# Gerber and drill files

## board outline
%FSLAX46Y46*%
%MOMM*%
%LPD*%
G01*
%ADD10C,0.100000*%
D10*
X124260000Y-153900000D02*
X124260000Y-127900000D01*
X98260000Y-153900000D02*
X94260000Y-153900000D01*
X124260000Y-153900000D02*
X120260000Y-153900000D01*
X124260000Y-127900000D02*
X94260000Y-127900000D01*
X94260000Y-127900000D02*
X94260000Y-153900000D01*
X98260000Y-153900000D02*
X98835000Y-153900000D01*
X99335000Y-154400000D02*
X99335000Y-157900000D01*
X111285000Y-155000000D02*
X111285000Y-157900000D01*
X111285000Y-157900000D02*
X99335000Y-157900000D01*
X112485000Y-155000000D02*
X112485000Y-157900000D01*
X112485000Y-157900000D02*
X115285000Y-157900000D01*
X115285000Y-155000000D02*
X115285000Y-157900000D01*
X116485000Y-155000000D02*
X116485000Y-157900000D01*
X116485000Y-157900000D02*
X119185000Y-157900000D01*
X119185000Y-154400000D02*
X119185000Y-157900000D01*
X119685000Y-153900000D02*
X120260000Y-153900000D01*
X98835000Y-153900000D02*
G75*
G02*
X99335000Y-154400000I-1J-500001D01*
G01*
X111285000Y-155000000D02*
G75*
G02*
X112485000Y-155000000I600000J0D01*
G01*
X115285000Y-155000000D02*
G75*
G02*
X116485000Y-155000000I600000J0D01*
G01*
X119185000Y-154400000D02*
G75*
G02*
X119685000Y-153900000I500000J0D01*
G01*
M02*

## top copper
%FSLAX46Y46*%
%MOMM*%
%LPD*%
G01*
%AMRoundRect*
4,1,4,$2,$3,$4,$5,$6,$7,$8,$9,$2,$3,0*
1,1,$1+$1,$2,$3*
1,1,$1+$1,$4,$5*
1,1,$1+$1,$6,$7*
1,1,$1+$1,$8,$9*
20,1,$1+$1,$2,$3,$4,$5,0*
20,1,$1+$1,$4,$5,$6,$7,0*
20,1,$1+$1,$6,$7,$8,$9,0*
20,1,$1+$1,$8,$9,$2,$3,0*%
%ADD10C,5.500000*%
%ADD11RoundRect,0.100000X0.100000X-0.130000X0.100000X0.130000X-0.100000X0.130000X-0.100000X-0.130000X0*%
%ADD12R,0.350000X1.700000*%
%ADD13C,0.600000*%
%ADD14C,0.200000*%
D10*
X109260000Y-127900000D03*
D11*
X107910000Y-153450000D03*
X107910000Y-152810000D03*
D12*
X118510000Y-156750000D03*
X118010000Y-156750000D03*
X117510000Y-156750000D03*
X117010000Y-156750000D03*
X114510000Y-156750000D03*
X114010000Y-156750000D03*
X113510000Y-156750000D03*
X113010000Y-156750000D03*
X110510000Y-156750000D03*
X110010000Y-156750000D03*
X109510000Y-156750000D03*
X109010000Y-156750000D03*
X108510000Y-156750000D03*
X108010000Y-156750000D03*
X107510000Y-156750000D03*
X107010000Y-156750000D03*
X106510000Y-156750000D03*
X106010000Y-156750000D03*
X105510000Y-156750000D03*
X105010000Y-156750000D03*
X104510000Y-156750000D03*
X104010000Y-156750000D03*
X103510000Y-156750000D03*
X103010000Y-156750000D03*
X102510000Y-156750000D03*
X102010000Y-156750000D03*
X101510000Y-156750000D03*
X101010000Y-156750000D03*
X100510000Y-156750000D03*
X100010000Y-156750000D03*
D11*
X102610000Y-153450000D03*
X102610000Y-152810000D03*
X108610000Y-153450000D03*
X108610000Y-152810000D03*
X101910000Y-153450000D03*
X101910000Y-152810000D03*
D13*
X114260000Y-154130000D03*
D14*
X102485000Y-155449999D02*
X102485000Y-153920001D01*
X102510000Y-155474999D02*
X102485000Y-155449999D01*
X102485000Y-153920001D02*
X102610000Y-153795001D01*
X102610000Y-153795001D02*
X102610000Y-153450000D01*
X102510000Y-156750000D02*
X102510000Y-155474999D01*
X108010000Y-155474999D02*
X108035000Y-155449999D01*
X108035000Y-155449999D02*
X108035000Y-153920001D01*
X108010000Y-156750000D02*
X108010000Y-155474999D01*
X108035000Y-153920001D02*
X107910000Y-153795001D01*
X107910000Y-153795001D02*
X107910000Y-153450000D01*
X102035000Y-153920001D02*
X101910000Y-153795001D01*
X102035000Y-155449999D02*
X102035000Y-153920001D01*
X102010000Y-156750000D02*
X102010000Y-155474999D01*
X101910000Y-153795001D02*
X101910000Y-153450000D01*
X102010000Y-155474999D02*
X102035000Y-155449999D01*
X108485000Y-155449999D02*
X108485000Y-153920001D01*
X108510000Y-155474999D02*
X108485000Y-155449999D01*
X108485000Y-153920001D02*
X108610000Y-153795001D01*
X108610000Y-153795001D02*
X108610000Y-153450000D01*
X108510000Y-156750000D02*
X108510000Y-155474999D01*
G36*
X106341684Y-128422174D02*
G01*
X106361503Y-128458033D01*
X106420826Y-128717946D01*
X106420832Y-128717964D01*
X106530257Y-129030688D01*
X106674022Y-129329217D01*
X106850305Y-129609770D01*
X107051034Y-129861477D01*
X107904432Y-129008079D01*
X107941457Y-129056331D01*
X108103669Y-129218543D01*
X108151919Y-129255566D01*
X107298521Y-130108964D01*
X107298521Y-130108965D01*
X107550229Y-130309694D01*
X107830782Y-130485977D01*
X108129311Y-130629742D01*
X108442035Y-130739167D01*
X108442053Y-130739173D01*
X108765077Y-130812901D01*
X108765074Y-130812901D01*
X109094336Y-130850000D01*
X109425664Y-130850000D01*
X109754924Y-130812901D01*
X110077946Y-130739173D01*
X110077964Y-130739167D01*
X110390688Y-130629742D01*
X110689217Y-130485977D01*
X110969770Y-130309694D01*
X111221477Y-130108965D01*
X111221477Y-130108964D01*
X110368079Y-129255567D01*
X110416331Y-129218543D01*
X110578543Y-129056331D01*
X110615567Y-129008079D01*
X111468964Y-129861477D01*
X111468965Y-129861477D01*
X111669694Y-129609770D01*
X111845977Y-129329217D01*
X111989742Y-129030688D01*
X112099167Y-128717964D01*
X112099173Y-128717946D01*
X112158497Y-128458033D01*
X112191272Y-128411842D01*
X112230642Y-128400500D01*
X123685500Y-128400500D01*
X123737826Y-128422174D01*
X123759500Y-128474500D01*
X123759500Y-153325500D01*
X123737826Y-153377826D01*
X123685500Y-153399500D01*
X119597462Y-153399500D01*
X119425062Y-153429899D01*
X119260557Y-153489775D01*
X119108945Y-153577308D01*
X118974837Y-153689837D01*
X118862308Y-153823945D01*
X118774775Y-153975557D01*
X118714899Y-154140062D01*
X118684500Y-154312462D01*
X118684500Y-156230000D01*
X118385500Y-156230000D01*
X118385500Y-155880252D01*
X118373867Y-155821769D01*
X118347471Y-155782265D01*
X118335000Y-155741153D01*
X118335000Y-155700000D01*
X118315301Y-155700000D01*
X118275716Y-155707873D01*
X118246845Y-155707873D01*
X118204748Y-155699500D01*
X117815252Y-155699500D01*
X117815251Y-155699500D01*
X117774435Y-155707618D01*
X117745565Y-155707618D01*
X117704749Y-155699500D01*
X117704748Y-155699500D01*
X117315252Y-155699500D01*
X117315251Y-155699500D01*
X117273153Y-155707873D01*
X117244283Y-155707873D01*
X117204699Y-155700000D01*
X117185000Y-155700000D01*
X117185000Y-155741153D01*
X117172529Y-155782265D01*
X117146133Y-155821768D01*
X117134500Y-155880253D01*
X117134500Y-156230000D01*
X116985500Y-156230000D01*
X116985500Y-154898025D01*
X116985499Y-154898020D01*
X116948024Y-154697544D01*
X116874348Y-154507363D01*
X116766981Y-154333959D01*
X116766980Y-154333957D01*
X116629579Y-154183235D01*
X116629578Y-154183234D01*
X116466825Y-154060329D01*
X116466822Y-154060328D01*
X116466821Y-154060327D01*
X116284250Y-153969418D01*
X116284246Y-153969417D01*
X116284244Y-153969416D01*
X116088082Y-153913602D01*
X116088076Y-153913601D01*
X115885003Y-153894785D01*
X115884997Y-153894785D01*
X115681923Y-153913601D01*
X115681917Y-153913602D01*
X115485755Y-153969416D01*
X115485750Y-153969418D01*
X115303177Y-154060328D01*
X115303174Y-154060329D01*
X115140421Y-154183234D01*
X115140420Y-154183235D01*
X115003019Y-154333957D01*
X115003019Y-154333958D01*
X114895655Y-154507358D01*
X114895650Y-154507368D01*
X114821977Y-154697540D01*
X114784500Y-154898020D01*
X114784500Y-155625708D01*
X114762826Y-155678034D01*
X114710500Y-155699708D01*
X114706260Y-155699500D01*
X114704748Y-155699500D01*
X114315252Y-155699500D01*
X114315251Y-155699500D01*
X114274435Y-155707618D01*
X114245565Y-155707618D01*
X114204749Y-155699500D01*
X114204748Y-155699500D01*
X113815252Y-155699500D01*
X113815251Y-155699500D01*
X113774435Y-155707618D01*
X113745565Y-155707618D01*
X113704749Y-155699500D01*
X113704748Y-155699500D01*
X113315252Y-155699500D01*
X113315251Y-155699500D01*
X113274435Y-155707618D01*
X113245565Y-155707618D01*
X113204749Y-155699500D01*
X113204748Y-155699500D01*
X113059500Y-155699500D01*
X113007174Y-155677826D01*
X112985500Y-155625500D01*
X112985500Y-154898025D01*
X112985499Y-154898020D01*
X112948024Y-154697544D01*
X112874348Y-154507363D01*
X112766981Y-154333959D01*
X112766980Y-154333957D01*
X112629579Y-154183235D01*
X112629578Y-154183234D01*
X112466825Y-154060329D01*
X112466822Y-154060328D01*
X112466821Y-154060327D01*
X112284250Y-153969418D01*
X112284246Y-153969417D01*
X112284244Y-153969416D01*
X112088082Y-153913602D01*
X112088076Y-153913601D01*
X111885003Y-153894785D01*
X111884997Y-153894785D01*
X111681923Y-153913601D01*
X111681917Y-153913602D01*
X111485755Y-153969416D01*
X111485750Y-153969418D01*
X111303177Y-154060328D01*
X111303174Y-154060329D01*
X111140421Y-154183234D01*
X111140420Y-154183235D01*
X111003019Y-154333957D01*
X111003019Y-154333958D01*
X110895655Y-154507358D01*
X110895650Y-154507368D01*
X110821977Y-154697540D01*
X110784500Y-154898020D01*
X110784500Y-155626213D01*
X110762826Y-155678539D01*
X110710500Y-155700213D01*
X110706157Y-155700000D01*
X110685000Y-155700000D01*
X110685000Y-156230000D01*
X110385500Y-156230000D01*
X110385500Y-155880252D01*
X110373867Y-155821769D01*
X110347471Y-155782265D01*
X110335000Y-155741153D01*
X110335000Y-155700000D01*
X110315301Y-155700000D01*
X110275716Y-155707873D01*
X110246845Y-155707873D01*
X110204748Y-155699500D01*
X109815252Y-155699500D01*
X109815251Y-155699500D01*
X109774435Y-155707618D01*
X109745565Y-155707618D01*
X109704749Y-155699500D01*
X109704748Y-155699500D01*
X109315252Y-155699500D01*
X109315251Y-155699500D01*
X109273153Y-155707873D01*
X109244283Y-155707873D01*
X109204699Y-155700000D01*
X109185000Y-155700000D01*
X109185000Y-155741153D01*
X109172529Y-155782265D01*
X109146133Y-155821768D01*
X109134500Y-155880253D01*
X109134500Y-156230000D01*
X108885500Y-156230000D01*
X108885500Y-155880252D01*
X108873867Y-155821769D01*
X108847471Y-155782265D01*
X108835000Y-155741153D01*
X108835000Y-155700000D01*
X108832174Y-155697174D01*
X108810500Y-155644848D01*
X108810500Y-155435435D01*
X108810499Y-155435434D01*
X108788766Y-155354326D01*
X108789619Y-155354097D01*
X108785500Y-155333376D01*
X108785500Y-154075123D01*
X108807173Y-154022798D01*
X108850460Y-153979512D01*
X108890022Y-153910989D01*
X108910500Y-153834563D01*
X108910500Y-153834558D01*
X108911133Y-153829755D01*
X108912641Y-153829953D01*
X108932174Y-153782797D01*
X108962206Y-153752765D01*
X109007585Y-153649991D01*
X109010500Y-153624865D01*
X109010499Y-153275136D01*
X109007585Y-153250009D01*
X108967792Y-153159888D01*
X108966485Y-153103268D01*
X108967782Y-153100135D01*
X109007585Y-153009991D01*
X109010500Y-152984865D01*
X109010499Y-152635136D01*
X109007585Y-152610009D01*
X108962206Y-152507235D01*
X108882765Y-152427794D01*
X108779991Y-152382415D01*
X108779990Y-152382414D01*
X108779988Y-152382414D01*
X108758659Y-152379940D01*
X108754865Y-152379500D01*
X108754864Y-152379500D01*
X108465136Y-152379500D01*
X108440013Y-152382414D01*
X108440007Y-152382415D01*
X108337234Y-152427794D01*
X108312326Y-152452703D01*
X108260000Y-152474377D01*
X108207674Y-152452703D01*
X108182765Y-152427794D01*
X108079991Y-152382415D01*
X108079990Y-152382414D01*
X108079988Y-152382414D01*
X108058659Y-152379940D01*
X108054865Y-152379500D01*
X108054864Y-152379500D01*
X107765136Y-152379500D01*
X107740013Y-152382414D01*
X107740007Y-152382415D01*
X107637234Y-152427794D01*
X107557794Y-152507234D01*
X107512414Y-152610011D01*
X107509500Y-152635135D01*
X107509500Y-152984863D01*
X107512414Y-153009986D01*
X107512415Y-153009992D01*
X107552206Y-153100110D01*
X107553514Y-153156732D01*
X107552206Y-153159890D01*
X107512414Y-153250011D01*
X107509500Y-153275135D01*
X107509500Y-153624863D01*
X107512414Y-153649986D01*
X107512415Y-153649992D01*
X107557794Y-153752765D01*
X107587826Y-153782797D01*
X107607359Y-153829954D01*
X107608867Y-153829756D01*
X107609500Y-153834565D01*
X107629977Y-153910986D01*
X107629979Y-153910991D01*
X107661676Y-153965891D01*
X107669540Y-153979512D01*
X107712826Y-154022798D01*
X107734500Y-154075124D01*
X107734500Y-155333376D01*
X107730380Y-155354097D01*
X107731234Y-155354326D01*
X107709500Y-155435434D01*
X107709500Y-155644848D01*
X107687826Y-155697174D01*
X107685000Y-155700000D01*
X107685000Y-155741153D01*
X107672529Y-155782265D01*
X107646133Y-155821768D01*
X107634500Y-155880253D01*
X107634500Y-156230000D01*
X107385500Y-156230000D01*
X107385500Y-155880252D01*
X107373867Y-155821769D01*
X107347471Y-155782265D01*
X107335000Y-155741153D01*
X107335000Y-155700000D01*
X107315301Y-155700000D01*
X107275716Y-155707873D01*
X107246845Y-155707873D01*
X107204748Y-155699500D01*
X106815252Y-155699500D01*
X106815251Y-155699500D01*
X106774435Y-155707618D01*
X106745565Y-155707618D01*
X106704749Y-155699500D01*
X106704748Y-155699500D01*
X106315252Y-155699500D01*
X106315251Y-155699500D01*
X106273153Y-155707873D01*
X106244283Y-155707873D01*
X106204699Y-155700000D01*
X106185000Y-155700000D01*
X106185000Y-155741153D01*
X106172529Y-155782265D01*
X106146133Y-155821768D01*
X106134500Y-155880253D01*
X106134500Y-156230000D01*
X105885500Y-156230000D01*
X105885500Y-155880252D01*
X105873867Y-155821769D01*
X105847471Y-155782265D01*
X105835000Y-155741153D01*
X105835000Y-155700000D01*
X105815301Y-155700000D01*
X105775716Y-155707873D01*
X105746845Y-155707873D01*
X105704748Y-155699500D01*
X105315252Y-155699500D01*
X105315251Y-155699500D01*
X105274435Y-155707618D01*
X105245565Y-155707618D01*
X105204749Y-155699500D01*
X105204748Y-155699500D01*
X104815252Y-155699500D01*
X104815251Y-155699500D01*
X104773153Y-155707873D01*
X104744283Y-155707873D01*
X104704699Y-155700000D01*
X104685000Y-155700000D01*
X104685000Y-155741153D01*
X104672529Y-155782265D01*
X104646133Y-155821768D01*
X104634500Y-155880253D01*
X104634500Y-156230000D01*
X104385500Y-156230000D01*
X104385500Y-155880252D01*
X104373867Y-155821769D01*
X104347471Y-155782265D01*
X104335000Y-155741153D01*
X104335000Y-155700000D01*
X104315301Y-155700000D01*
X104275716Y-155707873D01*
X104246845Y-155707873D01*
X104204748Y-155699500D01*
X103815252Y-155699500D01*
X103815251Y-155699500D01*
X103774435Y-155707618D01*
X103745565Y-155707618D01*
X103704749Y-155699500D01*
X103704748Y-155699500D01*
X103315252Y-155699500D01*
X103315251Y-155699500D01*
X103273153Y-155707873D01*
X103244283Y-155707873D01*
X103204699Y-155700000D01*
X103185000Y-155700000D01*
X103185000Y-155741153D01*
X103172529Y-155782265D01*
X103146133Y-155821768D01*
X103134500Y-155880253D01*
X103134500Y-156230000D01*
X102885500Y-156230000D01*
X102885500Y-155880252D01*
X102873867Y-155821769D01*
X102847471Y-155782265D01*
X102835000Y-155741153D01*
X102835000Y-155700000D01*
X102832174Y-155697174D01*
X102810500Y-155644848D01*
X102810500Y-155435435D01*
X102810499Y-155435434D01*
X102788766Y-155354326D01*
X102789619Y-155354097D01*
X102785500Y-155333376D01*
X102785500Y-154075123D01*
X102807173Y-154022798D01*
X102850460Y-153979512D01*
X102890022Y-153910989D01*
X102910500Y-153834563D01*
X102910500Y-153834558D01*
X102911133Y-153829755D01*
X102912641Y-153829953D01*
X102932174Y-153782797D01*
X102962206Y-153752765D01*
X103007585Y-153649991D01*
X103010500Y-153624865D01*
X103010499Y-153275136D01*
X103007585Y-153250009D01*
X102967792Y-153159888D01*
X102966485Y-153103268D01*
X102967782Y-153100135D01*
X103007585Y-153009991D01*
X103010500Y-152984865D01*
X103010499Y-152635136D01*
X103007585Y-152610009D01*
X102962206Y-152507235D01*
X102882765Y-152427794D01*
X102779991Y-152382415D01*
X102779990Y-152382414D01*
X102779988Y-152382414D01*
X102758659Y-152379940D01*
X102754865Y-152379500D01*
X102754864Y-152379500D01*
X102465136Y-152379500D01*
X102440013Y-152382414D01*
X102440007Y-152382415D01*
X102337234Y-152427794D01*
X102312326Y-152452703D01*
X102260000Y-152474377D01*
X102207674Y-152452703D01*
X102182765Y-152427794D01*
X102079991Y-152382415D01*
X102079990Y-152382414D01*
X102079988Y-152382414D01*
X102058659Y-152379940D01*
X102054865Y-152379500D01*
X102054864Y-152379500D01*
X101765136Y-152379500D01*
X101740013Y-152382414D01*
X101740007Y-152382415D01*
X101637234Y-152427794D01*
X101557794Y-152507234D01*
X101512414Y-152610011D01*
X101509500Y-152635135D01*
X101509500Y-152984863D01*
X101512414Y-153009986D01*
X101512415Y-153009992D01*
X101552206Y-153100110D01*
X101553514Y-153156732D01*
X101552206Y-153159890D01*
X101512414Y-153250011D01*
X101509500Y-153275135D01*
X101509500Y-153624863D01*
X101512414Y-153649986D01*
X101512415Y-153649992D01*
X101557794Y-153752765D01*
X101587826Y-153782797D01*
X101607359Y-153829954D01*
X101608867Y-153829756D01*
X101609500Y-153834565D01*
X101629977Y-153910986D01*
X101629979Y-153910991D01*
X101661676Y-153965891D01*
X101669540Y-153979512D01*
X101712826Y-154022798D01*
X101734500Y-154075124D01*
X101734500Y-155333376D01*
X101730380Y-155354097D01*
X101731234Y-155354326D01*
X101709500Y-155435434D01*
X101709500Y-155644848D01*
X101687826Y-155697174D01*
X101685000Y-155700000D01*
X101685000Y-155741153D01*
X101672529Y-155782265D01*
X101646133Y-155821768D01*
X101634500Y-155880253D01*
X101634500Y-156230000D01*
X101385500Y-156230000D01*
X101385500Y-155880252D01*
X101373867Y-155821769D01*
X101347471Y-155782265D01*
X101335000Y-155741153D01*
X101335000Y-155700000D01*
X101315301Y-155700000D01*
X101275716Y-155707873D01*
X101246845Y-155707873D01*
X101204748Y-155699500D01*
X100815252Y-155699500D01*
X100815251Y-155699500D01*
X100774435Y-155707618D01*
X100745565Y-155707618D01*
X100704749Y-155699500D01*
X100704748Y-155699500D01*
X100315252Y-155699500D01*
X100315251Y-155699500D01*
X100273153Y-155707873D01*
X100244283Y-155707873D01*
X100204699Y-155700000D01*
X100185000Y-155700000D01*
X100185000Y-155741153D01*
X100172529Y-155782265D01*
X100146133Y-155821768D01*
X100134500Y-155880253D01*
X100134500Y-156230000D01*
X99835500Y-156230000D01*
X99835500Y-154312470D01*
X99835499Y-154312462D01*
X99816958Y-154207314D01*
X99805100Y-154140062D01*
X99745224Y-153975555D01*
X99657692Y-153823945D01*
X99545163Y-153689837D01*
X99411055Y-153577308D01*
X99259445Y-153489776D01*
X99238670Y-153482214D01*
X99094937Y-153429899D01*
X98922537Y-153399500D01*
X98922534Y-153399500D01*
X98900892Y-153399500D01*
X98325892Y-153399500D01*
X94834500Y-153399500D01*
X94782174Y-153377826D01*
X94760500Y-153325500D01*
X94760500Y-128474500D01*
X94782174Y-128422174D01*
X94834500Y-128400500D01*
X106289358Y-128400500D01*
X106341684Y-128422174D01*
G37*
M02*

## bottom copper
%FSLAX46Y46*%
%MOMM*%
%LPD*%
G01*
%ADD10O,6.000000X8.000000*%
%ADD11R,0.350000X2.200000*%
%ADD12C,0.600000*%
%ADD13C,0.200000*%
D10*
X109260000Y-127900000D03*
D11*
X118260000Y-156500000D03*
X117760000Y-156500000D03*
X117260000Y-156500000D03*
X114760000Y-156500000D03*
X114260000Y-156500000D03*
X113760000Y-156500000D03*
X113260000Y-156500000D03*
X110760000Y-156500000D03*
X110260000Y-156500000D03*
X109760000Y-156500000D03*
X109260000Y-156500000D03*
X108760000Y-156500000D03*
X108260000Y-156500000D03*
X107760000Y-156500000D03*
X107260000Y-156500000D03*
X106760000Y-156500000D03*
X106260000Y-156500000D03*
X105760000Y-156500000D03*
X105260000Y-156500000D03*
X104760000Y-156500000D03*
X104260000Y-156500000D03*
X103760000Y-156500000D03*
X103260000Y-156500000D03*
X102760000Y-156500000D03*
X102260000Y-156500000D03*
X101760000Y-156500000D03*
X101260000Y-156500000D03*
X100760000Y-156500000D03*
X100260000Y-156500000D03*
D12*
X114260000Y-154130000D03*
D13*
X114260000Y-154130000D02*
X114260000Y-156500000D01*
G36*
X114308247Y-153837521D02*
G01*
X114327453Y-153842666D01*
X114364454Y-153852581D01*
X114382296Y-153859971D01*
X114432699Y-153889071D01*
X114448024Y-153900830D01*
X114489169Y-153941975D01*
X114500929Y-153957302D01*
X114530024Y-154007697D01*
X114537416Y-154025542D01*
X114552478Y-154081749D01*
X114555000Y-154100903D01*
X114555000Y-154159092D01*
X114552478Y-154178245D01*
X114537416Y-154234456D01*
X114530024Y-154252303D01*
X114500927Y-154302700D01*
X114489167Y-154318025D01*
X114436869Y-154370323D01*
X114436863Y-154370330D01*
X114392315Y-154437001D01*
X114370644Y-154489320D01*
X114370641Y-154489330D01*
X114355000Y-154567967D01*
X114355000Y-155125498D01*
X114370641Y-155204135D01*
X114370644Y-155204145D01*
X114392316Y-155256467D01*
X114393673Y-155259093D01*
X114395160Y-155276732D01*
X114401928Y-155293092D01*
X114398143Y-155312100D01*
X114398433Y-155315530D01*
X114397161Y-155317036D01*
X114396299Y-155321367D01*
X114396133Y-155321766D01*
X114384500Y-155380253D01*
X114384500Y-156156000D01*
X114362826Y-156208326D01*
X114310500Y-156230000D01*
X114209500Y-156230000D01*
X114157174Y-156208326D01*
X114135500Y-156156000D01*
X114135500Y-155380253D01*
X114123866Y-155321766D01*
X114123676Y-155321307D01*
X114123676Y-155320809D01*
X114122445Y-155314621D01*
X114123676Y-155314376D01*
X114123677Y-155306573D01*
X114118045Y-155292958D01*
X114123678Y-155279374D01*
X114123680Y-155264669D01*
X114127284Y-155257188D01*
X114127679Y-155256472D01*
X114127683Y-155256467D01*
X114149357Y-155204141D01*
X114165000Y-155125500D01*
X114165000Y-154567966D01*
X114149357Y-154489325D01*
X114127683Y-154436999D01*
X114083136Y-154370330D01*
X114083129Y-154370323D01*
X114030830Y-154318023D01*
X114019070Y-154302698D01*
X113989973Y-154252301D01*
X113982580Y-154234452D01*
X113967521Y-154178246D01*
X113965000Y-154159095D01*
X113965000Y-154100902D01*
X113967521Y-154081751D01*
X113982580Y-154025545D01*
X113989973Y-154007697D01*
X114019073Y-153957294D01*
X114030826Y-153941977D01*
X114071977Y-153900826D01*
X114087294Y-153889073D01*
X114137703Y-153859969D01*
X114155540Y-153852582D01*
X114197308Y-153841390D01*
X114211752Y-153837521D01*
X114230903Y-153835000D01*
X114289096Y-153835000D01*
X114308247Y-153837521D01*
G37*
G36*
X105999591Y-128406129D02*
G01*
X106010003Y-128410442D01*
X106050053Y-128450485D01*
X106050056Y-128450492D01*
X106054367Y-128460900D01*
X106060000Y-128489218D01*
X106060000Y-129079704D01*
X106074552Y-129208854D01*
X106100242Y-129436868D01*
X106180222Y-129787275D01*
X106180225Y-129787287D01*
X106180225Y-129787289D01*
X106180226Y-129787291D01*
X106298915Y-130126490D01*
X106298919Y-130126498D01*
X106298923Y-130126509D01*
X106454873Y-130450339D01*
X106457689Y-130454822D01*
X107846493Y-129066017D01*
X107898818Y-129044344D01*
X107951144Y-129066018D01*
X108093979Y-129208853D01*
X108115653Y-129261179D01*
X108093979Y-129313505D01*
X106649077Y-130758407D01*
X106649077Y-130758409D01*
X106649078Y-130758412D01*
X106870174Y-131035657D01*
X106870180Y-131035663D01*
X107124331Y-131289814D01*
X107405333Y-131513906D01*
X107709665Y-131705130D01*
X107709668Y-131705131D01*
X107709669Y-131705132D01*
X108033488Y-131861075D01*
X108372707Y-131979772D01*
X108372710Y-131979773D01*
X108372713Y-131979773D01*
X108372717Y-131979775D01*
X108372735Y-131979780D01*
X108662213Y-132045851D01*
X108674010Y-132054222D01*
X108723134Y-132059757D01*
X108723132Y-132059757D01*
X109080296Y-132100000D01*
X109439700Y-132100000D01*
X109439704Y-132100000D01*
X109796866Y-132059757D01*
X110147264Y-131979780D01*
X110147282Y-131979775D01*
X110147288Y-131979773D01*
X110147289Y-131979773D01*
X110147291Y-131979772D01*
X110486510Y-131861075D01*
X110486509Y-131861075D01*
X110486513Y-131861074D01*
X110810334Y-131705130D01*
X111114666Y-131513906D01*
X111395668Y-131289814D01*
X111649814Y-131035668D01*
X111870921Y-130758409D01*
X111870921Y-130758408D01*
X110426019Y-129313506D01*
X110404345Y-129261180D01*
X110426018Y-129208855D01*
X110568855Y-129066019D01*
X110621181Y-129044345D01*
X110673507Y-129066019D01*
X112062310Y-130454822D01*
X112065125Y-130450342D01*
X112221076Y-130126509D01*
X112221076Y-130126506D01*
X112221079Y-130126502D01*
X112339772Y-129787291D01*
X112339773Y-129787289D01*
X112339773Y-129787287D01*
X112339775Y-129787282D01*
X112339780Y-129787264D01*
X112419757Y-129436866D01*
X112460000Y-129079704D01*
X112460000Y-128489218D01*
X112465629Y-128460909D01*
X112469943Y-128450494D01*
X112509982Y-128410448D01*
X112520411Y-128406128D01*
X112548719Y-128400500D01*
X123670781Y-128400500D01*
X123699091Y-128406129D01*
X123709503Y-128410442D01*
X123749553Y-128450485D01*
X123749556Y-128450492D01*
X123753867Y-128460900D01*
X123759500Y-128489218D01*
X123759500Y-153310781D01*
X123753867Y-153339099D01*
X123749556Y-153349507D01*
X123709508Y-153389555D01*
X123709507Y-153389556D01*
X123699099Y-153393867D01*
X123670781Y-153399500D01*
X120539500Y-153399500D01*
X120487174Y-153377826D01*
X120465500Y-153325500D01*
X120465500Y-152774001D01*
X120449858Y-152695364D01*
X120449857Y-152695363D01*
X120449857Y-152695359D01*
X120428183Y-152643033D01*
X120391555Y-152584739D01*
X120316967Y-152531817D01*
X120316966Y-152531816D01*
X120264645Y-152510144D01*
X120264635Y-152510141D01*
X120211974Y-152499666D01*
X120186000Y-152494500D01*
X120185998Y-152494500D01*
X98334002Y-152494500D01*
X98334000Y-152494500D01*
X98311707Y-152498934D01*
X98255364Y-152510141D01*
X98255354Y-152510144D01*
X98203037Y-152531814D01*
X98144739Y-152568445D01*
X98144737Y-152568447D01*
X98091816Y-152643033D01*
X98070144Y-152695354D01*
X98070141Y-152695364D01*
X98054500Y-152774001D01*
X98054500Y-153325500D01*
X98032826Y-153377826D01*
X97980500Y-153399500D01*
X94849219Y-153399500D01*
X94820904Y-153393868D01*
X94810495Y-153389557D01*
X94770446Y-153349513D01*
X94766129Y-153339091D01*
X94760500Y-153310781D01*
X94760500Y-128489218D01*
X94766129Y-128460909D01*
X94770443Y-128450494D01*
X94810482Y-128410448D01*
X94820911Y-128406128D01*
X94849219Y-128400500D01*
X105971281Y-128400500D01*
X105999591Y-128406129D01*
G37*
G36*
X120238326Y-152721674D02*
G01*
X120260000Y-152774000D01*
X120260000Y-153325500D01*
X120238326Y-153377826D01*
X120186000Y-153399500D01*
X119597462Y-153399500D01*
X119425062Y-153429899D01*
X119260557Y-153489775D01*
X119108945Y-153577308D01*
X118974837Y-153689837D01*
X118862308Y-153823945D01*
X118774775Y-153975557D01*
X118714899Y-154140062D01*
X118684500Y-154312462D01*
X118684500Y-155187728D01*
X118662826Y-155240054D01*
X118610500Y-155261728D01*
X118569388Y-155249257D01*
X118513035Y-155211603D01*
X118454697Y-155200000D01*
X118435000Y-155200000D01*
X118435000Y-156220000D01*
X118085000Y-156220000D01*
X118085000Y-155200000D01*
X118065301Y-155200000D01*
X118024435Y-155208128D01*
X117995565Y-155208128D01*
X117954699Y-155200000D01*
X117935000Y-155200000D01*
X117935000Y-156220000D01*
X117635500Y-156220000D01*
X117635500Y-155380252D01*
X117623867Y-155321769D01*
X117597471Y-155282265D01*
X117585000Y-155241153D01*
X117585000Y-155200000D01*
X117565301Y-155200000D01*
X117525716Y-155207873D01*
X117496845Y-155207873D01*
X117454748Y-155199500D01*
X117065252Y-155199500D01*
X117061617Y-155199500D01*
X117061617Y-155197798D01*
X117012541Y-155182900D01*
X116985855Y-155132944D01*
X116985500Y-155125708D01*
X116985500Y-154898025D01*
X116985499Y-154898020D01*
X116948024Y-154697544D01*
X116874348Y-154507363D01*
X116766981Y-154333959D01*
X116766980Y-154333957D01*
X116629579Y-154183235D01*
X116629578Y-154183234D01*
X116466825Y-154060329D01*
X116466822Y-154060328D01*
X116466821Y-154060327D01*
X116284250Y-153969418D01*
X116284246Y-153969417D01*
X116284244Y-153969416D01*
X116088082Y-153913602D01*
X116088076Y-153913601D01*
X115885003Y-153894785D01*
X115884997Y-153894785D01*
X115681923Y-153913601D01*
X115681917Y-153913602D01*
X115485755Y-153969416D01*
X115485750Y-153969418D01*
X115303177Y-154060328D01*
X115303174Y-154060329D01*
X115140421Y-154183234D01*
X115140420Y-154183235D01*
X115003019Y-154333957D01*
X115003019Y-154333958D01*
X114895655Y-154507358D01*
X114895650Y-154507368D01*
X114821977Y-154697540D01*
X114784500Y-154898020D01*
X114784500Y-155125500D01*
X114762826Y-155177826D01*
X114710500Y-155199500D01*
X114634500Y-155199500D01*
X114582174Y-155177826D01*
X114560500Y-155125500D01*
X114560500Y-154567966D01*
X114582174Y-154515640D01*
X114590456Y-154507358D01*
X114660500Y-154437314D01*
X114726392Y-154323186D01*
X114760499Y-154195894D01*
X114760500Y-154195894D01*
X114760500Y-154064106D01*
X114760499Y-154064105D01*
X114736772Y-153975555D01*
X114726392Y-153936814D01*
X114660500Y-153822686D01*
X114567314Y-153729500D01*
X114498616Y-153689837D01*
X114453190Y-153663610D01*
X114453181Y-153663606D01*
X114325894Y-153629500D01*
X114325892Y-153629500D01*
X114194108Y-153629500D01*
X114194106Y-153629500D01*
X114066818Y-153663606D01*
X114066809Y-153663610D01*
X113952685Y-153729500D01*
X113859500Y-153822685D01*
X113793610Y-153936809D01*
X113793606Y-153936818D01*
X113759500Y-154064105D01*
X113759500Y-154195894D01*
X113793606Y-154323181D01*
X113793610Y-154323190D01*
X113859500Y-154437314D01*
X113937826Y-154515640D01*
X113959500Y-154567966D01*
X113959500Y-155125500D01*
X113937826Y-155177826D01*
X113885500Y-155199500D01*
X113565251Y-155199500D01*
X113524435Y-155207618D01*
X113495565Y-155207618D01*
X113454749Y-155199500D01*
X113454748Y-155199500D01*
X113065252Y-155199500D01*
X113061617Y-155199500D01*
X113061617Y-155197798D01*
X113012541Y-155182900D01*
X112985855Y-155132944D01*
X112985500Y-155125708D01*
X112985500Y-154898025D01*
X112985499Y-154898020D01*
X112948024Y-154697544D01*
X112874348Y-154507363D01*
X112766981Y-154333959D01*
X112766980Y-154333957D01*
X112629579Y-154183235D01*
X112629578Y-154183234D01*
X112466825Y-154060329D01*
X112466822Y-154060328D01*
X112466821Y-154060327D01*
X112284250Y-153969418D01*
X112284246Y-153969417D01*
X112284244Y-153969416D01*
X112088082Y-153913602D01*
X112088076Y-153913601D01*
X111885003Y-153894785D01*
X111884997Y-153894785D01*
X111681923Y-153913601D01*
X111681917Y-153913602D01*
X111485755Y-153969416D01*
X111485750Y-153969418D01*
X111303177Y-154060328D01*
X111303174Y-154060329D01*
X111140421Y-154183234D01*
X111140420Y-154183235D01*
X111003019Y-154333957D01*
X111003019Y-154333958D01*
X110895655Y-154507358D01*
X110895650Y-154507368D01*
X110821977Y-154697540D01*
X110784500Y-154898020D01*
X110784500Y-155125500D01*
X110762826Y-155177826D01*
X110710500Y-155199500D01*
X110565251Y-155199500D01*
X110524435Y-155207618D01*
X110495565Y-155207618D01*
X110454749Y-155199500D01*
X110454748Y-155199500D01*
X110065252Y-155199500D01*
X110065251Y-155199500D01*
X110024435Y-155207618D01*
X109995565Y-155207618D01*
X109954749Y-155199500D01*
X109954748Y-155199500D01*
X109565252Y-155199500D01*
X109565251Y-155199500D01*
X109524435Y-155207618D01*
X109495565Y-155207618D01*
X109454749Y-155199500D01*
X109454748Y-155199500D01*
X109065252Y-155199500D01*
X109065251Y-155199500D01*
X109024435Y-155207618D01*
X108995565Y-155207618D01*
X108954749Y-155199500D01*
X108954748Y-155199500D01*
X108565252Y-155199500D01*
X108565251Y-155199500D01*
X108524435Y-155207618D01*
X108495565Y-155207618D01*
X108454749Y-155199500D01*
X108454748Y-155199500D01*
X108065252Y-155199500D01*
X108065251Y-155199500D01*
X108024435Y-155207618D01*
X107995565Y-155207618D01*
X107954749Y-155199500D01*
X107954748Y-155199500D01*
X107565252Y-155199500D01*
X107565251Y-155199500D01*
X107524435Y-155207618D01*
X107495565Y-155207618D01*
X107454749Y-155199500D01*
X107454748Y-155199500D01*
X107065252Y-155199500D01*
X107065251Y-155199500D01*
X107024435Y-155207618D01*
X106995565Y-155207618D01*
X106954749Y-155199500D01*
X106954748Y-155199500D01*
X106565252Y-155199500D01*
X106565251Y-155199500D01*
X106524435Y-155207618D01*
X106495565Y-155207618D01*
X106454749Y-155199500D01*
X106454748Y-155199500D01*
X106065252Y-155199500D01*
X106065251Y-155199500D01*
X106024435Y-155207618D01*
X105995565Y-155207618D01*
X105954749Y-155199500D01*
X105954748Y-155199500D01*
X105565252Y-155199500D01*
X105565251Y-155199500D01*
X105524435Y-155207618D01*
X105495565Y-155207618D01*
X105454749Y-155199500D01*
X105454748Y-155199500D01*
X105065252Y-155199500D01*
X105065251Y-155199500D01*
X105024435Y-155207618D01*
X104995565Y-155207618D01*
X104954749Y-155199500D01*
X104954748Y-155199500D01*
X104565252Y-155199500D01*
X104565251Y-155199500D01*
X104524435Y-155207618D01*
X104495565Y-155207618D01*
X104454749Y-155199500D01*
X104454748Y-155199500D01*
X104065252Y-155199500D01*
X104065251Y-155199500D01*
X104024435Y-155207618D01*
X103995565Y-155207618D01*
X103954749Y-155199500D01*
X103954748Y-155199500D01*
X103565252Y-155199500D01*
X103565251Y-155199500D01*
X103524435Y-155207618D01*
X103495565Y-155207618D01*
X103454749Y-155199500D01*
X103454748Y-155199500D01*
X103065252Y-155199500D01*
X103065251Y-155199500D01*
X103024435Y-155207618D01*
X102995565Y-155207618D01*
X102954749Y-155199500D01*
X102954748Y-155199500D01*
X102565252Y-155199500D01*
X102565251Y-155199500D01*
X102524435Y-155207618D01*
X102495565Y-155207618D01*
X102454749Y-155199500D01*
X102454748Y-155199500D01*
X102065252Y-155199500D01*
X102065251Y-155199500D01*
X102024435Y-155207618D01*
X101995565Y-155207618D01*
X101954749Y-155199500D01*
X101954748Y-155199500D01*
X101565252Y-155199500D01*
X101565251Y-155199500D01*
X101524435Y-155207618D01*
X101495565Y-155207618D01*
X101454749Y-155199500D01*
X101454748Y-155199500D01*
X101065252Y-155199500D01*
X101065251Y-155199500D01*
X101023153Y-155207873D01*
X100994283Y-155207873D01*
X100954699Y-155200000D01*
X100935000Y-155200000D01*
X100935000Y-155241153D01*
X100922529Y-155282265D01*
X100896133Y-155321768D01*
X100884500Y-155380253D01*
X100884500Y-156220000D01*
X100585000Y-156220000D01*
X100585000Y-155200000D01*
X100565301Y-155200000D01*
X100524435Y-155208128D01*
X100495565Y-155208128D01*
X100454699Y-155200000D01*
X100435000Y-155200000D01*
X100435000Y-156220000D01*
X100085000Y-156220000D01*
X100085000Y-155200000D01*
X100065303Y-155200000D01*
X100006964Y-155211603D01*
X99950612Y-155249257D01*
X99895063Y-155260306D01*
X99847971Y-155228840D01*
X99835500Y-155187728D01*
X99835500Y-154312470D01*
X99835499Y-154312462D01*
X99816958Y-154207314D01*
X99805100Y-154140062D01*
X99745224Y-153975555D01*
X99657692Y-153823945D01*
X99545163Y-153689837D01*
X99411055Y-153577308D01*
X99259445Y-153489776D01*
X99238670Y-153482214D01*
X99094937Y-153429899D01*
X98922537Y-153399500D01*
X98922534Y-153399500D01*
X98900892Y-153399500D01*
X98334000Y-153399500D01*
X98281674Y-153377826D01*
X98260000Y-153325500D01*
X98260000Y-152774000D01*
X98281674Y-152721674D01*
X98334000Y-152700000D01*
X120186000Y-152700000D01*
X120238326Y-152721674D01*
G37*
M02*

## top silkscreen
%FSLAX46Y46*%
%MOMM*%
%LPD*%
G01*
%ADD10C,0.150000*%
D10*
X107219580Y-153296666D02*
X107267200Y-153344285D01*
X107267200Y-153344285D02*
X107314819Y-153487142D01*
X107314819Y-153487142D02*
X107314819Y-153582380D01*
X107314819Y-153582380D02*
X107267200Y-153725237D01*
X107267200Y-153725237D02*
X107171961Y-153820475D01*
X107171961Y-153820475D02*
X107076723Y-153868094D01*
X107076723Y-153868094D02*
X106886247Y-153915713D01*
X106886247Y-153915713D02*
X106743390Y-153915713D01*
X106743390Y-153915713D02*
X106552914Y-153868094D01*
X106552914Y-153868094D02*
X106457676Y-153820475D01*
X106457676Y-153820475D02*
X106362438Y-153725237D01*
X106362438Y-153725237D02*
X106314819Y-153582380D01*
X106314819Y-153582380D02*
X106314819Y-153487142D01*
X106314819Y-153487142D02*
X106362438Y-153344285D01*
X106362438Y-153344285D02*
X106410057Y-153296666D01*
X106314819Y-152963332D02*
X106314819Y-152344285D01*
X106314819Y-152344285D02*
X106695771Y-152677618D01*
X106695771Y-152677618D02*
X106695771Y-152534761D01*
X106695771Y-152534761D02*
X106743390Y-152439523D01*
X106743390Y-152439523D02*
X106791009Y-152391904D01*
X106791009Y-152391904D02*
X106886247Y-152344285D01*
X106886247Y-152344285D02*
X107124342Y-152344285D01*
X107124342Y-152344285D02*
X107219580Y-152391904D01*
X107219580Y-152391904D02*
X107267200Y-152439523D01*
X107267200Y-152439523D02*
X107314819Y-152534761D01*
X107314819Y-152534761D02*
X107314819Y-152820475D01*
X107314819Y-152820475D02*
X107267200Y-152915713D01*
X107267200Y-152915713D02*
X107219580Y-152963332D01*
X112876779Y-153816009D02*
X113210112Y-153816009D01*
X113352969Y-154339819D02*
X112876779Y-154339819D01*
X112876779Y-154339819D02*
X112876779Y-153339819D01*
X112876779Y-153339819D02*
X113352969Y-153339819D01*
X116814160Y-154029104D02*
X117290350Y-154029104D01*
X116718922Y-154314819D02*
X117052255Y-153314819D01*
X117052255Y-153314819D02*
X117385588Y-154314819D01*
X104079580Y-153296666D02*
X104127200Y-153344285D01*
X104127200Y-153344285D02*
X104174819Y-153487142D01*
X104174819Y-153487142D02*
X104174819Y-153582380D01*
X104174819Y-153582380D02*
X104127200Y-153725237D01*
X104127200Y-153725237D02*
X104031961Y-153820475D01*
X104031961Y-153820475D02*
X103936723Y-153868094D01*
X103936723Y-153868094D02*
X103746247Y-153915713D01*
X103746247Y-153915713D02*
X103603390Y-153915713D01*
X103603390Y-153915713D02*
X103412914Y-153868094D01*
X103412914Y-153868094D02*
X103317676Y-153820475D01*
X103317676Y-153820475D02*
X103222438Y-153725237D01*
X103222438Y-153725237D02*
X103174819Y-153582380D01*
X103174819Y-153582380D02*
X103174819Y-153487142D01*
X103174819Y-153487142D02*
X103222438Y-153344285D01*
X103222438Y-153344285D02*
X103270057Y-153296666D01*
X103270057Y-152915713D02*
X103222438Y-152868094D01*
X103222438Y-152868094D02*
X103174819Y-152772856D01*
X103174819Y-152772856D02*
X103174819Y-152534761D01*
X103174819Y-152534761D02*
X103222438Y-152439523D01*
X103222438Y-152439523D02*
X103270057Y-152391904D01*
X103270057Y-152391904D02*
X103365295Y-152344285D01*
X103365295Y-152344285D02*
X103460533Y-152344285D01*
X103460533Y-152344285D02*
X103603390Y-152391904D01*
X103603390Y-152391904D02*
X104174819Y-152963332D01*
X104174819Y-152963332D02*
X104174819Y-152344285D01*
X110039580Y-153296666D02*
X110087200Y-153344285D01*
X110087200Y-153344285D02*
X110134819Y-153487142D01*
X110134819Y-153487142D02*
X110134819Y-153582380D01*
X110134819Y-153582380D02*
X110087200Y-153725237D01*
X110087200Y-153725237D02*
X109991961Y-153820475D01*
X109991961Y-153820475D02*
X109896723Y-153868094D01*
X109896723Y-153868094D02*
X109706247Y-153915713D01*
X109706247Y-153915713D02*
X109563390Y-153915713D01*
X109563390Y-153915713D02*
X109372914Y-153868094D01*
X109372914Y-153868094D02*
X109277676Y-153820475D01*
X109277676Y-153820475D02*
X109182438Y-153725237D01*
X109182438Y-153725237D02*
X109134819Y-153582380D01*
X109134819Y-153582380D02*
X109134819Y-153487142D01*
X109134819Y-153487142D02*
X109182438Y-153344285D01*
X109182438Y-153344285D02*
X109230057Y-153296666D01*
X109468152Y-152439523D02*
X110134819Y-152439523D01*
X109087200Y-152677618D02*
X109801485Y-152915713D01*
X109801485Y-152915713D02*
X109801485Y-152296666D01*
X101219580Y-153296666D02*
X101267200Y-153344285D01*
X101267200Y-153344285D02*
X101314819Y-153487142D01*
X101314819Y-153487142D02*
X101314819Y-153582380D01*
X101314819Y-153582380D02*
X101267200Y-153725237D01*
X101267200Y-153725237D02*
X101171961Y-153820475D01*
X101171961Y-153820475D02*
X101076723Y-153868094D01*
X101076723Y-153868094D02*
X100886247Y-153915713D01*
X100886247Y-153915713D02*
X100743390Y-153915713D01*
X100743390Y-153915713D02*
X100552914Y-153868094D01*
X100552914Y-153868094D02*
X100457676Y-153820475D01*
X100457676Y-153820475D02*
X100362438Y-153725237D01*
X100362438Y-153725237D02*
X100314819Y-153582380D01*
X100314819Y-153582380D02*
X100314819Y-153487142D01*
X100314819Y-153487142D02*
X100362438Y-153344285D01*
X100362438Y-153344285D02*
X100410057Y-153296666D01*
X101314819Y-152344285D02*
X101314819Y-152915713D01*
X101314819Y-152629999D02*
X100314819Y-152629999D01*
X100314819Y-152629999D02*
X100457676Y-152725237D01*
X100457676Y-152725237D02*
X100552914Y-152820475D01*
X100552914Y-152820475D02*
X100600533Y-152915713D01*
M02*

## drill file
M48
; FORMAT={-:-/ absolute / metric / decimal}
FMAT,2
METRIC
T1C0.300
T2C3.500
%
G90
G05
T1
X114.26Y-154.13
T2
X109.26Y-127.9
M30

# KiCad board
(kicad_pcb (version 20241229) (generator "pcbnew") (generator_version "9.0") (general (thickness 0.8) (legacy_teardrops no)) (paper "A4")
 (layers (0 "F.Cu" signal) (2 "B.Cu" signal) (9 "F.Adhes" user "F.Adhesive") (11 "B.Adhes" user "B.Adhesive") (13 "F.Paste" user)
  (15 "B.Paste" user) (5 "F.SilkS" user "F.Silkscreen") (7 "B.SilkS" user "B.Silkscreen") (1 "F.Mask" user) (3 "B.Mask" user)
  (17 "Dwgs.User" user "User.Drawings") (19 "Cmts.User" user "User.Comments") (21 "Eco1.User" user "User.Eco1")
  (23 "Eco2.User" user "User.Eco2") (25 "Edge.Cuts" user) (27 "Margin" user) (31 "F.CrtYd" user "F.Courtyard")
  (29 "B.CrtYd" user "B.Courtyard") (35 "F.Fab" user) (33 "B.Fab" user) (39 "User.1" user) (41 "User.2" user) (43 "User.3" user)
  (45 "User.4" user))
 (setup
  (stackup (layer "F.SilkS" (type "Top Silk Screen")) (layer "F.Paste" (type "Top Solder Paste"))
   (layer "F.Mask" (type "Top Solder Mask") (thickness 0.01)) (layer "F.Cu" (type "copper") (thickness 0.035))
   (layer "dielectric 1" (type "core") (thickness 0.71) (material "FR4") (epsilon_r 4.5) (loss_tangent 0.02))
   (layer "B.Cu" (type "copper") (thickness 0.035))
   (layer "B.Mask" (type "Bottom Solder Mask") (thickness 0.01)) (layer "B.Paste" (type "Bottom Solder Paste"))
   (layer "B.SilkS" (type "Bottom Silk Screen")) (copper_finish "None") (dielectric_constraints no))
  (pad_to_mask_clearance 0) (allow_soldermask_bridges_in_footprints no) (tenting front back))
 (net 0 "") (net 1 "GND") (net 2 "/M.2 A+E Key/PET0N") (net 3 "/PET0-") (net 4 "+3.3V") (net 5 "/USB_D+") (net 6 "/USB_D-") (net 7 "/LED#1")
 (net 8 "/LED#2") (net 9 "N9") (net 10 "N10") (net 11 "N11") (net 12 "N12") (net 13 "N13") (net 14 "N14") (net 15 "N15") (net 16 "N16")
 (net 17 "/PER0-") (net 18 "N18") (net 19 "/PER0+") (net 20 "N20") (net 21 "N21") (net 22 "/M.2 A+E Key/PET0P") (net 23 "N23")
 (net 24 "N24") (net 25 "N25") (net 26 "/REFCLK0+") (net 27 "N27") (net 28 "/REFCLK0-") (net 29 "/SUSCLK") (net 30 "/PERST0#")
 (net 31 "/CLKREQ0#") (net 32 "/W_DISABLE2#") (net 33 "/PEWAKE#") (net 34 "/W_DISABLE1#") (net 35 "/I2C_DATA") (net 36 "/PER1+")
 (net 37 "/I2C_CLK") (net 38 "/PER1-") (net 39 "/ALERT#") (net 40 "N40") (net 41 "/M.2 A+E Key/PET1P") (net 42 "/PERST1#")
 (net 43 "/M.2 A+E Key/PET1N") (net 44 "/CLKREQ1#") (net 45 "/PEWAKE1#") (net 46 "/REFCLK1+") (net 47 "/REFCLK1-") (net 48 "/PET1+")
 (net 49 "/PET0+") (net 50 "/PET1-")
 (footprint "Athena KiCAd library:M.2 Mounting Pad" (layer "F.Cu") (at 109.26 127.9)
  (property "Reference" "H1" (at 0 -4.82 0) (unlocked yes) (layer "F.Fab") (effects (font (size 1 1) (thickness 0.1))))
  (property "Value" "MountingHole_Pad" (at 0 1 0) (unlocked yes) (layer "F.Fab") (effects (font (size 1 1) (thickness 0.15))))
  (pad "1" thru_hole circle (at 0 0) (size 5.5 5.5) (drill 3.5) (layers "*.Cu" "*.Mask") (remove_unused_layers no) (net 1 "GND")
   (padstack (mode front_inner_back)
    (layer "Inner" (shape circle) (size 5.5 5.5) (zone_connect -1))
    (layer "B.Cu" (shape oval) (size 6 8) (thermal_bridge_angle 45) (zone_connect -1)))))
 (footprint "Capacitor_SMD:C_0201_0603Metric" (layer "F.Cu") (at 107.91 153.13 90)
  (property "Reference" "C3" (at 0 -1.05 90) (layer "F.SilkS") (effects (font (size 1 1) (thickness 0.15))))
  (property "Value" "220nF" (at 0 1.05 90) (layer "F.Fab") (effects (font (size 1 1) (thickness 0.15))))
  (pad "" smd roundrect (at -0.345 0 90) (size 0.318 0.36) (layers "F.Paste") (roundrect_rratio 0.25))
  (pad "" smd roundrect (at 0.345 0 90) (size 0.318 0.36) (layers "F.Paste") (roundrect_rratio 0.25))
  (pad "1" smd roundrect (at -0.32 0 90) (size 0.46 0.4) (layers "F.Cu" "F.Mask") (roundrect_rratio 0.25) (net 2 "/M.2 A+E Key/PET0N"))
  (pad "2" smd roundrect (at 0.32 0 90) (size 0.46 0.4) (layers "F.Cu" "F.Mask") (roundrect_rratio 0.25) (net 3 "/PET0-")))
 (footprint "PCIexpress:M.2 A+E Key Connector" (layer "F.Cu") (at 109.26 156.79)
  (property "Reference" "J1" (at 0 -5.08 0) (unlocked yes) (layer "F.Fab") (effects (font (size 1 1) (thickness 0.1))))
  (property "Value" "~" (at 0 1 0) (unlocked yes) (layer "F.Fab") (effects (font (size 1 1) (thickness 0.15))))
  (fp_line (start -11 -2.89) (end -10.425 -2.89) (stroke (width 0.1) (type default)) (layer "Edge.Cuts"))
  (fp_line (start -9.925 -2.39) (end -9.925 1.11) (stroke (width 0.1) (type default)) (layer "Edge.Cuts"))
  (fp_line (start 2.025 -1.79) (end 2.025 1.11) (stroke (width 0.1) (type default)) (layer "Edge.Cuts"))
  (fp_line (start 2.025 1.11) (end -9.925 1.11) (stroke (width 0.1) (type default)) (layer "Edge.Cuts"))
  (fp_line (start 3.225 -1.79) (end 3.225 1.11) (stroke (width 0.1) (type default)) (layer "Edge.Cuts"))
  (fp_line (start 3.225 1.11) (end 6.025 1.11) (stroke (width 0.1) (type default)) (layer "Edge.Cuts"))
  (fp_line (start 6.025 -1.79) (end 6.025 1.11) (stroke (width 0.1) (type default)) (layer "Edge.Cuts"))
  (fp_line (start 7.225 -1.79) (end 7.225 1.11) (stroke (width 0.1) (type default)) (layer "Edge.Cuts"))
  (fp_line (start 7.225 1.11) (end 9.925 1.11) (stroke (width 0.1) (type default)) (layer "Edge.Cuts"))
  (fp_line (start 9.925 -2.39) (end 9.925 1.11) (stroke (width 0.1) (type default)) (layer "Edge.Cuts"))
  (fp_line (start 10.425 -2.89) (end 11 -2.89) (stroke (width 0.1) (type default)) (layer "Edge.Cuts"))
  (fp_arc (start -10.425 -2.89) (mid -10.071447 -2.743553) (end -9.925 -2.39) (stroke (width 0.1) (type default)) (layer "Edge.Cuts"))
  (fp_arc (start 2.025 -1.79) (mid 2.625 -2.39) (end 3.225 -1.79) (stroke (width 0.1) (type default)) (layer "Edge.Cuts"))
  (fp_arc (start 6.025 -1.79) (mid 6.625 -2.39) (end 7.225 -1.79) (stroke (width 0.1) (type default)) (layer "Edge.Cuts"))
  (fp_arc (start 9.925 -2.39) (mid 10.071447 -2.743553) (end 10.425 -2.89) (stroke (width 0.1) (type default)) (layer "Edge.Cuts"))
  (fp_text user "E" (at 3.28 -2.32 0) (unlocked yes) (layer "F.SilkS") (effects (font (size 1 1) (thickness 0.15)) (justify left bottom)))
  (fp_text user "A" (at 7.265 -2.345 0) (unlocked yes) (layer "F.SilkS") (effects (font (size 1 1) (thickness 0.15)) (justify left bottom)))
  (pad "1" smd rect (at 9.25 -0.04 180) (size 0.35 1.7) (layers "F.Cu") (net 1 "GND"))
  (pad "2" smd rect (at 9 -0.29 180) (size 0.35 2.2) (layers "B.Cu") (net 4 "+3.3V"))
  (pad "3" smd rect (at 8.75 -0.04 180) (size 0.35 1.7) (layers "F.Cu") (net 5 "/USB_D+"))
  (pad "4" smd rect (at 8.5 -0.29 180) (size 0.35 2.2) (layers "B.Cu") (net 4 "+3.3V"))
  (pad "5" smd rect (at 8.25 -0.04 180) (size 0.35 1.7) (layers "F.Cu") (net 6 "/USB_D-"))
  (pad "6" smd rect (at 8 -0.29 180) (size 0.35 2.2) (layers "B.Cu") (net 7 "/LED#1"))
  (pad "7" smd rect (at 7.75 -0.04 180) (size 0.35 1.7) (layers "F.Cu") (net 1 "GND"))
  (pad "16" smd rect (at 5.5 -0.29 180) (size 0.35 2.2) (layers "B.Cu") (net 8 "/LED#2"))
  (pad "17" smd rect (at 5.25 -0.04 180) (size 0.35 1.7) (layers "F.Cu") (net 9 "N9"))
  (pad "18" smd rect (at 5 -0.29 180) (size 0.35 2.2) (layers "B.Cu") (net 1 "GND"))
  (pad "19" smd rect (at 4.75 -0.04 180) (size 0.35 1.7) (layers "F.Cu") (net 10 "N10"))
  (pad "20" smd rect (at 4.5 -0.29 180) (size 0.35 2.2) (layers "B.Cu") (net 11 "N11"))
  (pad "21" smd rect (at 4.25 -0.04 180) (size 0.35 1.7) (layers "F.Cu") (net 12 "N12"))
  (pad "22" smd rect (at 4 -0.29 180) (size 0.35 2.2) (layers "B.Cu") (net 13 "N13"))
  (pad "23" smd rect (at 3.75 -0.04 180) (size 0.35 1.7) (layers "F.Cu") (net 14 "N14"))
  (pad "32" smd rect (at 1.5 -0.29 180) (size 0.35 2.2) (layers "B.Cu") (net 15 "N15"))
  (pad "33" smd rect (at 1.25 -0.04 180) (size 0.35 1.7) (layers "F.Cu") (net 1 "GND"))
  (pad "34" smd rect (at 1 -0.29 180) (size 0.35 2.2) (layers "B.Cu") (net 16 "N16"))
  (pad "35" smd rect (at 0.75 -0.04 180) (size 0.35 1.7) (layers "F.Cu") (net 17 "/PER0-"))
  (pad "36" smd rect (at 0.5 -0.29 180) (size 0.35 2.2) (layers "B.Cu") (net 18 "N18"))
  (pad "37" smd rect (at 0.25 -0.04 180) (size 0.35 1.7) (layers "F.Cu") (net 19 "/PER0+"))
  (pad "38" smd rect (at 0 -0.29 180) (size 0.35 2.2) (layers "B.Cu") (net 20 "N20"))
  (pad "39" smd rect (at -0.25 -0.04 180) (size 0.35 1.7) (layers "F.Cu") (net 1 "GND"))
  (pad "40" smd rect (at -0.5 -0.29 180) (size 0.35 2.2) (layers "B.Cu") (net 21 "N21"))
  (pad "41" smd rect (at -0.75 -0.04 180) (size 0.35 1.7) (layers "F.Cu") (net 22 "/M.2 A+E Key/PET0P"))
  (pad "42" smd rect (at -1 -0.29 180) (size 0.35 2.2) (layers "B.Cu") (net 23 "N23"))
  (pad "43" smd rect (at -1.25 -0.04 180) (size 0.35 1.7) (layers "F.Cu") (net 2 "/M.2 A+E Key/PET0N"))
  (pad "44" smd rect (at -1.5 -0.29 180) (size 0.35 2.2) (layers "B.Cu") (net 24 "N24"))
  (pad "45" smd rect (at -1.75 -0.04 180) (size 0.35 1.7) (layers "F.Cu") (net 1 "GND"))
  (pad "46" smd rect (at -2 -0.29 180) (size 0.35 2.2) (layers "B.Cu") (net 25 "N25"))
  (pad "47" smd rect (at -2.25 -0.04 180) (size 0.35 1.7) (layers "F.Cu") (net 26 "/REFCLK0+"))
  (pad "48" smd rect (at -2.5 -0.29 180) (size 0.35 2.2) (layers "B.Cu") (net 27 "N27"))
  (pad "49" smd rect (at -2.75 -0.04 180) (size 0.35 1.7) (layers "F.Cu") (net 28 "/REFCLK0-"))
  (pad "50" smd rect (at -3 -0.29 180) (size 0.35 2.2) (layers "B.Cu") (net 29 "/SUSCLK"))
  (pad "51" smd rect (at -3.25 -0.04 180) (size 0.35 1.7) (layers "F.Cu") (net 1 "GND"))
  (pad "52" smd rect (at -3.5 -0.29 180) (size 0.35 2.2) (layers "B.Cu") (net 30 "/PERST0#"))
  (pad "53" smd rect (at -3.75 -0.04 180) (size 0.35 1.7) (layers "F.Cu") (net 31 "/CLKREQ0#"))
  (pad "54" smd rect (at -4 -0.29 180) (size 0.35 2.2) (layers "B.Cu") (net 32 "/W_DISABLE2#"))
  (pad "55" smd rect (at -4.25 -0.04 180) (size 0.35 1.7) (layers "F.Cu") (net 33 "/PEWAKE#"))
  (pad "56" smd rect (at -4.5 -0.29 180) (size 0.35 2.2) (layers "B.Cu") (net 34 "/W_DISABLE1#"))
  (pad "57" smd rect (at -4.75 -0.04 180) (size 0.35 1.7) (layers "F.Cu") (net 1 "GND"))
  (pad "58" smd rect (at -5 -0.29 180) (size 0.35 2.2) (layers "B.Cu") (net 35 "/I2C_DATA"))
  (pad "59" smd rect (at -5.25 -0.04 180) (size 0.35 1.7) (layers "F.Cu") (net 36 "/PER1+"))
  (pad "60" smd rect (at -5.5 -0.29 180) (size 0.35 2.2) (layers "B.Cu") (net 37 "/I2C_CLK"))
  (pad "61" smd rect (at -5.75 -0.04 180) (size 0.35 1.7) (layers "F.Cu") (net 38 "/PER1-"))
  (pad "62" smd rect (at -6 -0.29 180) (size 0.35 2.2) (layers "B.Cu") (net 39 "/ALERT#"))
  (pad "63" smd rect (at -6.25 -0.04 180) (size 0.35 1.7) (layers "F.Cu") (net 1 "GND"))
  (pad "64" smd rect (at -6.5 -0.29 180) (size 0.35 2.2) (layers "B.Cu") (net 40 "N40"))
  (pad "65" smd rect (at -6.75 -0.04 180) (size 0.35 1.7) (layers "F.Cu") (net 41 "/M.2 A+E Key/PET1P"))
  (pad "66" smd rect (at -7 -0.29 180) (size 0.35 2.2) (layers "B.Cu") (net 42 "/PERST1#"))
  (pad "67" smd rect (at -7.25 -0.04 180) (size 0.35 1.7) (layers "F.Cu") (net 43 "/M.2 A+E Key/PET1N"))
  (pad "68" smd rect (at -7.5 -0.29 180) (size 0.35 2.2) (layers "B.Cu") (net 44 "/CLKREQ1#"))
  (pad "69" smd rect (at -7.75 -0.04 180) (size 0.35 1.7) (layers "F.Cu") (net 1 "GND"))
  (pad "70" smd rect (at -8 -0.29 180) (size 0.35 2.2) (layers "B.Cu") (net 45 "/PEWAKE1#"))
  (pad "71" smd rect (at -8.25 -0.04 180) (size 0.35 1.7) (layers "F.Cu") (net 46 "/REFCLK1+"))
  (pad "72" smd rect (at -8.5 -0.29 180) (size 0.35 2.2) (layers "B.Cu") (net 4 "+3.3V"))
  (pad "73" smd rect (at -8.75 -0.04 180) (size 0.35 1.7) (layers "F.Cu") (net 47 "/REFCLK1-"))
  (pad "74" smd rect (at -9 -0.29 180) (size 0.35 2.2) (layers "B.Cu") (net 4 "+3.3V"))
  (pad "75" smd rect (at -9.25 -0.04 180) (size 0.35 1.7) (layers "F.Cu") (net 1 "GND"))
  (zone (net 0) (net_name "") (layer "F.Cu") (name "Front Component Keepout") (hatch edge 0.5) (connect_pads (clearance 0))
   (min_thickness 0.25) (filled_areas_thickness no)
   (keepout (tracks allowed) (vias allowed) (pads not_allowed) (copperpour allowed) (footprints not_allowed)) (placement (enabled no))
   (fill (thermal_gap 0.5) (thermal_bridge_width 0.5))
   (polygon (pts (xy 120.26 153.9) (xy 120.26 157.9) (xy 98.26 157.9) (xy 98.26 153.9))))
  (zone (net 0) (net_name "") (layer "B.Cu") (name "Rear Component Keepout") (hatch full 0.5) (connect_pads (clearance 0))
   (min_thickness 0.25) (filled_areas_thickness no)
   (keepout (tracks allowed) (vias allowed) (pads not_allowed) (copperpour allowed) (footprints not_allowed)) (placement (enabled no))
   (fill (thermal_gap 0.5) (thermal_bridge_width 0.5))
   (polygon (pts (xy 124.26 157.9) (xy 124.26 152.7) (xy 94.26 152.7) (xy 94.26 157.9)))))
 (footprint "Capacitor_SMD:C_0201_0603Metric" (layer "F.Cu") (at 102.61 153.13 90)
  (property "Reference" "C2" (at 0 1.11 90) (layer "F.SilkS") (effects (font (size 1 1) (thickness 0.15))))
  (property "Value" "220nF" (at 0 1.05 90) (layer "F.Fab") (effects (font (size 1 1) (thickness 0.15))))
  (pad "" smd roundrect (at -0.345 0 90) (size 0.318 0.36) (layers "F.Paste") (roundrect_rratio 0.25))
  (pad "" smd roundrect (at 0.345 0 90) (size 0.318 0.36) (layers "F.Paste") (roundrect_rratio 0.25))
  (pad "1" smd roundrect (at -0.32 0 90) (size 0.46 0.4) (layers "F.Cu" "F.Mask") (roundrect_rratio 0.25) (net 41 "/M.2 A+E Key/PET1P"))
  (pad "2" smd roundrect (at 0.32 0 90) (size 0.46 0.4) (layers "F.Cu" "F.Mask") (roundrect_rratio 0.25) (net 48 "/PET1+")))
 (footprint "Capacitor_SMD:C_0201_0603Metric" (layer "F.Cu") (at 108.61 153.13 90)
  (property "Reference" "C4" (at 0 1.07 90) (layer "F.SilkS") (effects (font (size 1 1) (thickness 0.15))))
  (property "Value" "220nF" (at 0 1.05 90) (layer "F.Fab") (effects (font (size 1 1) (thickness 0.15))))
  (pad "" smd roundrect (at -0.345 0 90) (size 0.318 0.36) (layers "F.Paste") (roundrect_rratio 0.25))
  (pad "" smd roundrect (at 0.345 0 90) (size 0.318 0.36) (layers "F.Paste") (roundrect_rratio 0.25))
  (pad "1" smd roundrect (at -0.32 0 90) (size 0.46 0.4) (layers "F.Cu" "F.Mask") (roundrect_rratio 0.25) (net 22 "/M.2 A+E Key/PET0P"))
  (pad "2" smd roundrect (at 0.32 0 90) (size 0.46 0.4) (layers "F.Cu" "F.Mask") (roundrect_rratio 0.25) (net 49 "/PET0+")))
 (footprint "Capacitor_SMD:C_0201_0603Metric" (layer "F.Cu") (at 101.91 153.13 90)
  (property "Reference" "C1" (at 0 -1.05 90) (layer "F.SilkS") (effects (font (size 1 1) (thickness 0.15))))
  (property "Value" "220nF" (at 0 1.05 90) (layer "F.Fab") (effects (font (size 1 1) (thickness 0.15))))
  (pad "" smd roundrect (at -0.345 0 90) (size 0.318 0.36) (layers "F.Paste") (roundrect_rratio 0.25))
  (pad "" smd roundrect (at 0.345 0 90) (size 0.318 0.36) (layers "F.Paste") (roundrect_rratio 0.25))
  (pad "1" smd roundrect (at -0.32 0 90) (size 0.46 0.4) (layers "F.Cu" "F.Mask") (roundrect_rratio 0.25) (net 43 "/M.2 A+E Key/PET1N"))
  (pad "2" smd roundrect (at 0.32 0 90) (size 0.46 0.4) (layers "F.Cu" "F.Mask") (roundrect_rratio 0.25) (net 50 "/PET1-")))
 (gr_line (start 124.26 153.9) (end 124.26 127.9) (stroke (width 0.1) (type default)) (layer "Edge.Cuts"))
 (gr_line (start 98.26 153.9) (end 94.26 153.9) (stroke (width 0.1) (type default)) (layer "Edge.Cuts"))
 (gr_line (start 124.26 153.9) (end 120.26 153.9) (stroke (width 0.1) (type default)) (layer "Edge.Cuts"))
 (gr_line (start 124.26 127.9) (end 94.26 127.9) (stroke (width 0.1) (type default)) (layer "Edge.Cuts"))
 (gr_line (start 94.26 127.9) (end 94.26 153.9) (stroke (width 0.1) (type default)) (layer "Edge.Cuts"))
 (via (at 114.26 154.13) (size 0.6) (drill 0.3) (layers "F.Cu" "B.Cu") (free yes) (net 1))
 (segment (start 114.26 154.13) (end 114.26 156.5) (width 0.2) (layer "B.Cu") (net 1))
 (segment (start 102.485 155.449999) (end 102.485 153.920001) (width 0.2) (layer "F.Cu") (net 41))
 (segment (start 102.51 155.474999) (end 102.485 155.449999) (width 0.2) (layer "F.Cu") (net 41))
 (segment (start 102.485 153.920001) (end 102.61 153.795001) (width 0.2) (layer "F.Cu") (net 41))
 (segment (start 102.61 153.795001) (end 102.61 153.45) (width 0.2) (layer "F.Cu") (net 41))
 (segment (start 102.51 156.75) (end 102.51 155.474999) (width 0.2) (layer "F.Cu") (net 41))
 (segment (start 108.01 155.474999) (end 108.035 155.449999) (width 0.2) (layer "F.Cu") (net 2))
 (segment (start 108.035 155.449999) (end 108.035 153.920001) (width 0.2) (layer "F.Cu") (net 2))
 (segment (start 108.01 156.75) (end 108.01 155.474999) (width 0.2) (layer "F.Cu") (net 2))
 (segment (start 108.035 153.920001) (end 107.91 153.795001) (width 0.2) (layer "F.Cu") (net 2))
 (segment (start 107.91 153.795001) (end 107.91 153.45) (width 0.2) (layer "F.Cu") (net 2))
 (segment (start 102.035 153.920001) (end 101.91 153.795001) (width 0.2) (layer "F.Cu") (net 43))
 (segment (start 102.035 155.449999) (end 102.035 153.920001) (width 0.2) (layer "F.Cu") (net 43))
 (segment (start 102.01 156.75) (end 102.01 155.474999) (width 0.2) (layer "F.Cu") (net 43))
 (segment (start 101.91 153.795001) (end 101.91 153.45) (width 0.2) (layer "F.Cu") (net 43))
 (segment (start 102.01 155.474999) (end 102.035 155.449999) (width 0.2) (layer "F.Cu") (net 43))
 (segment (start 108.485 155.449999) (end 108.485 153.920001) (width 0.2) (layer "F.Cu") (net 22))
 (segment (start 108.51 155.474999) (end 108.485 155.449999) (width 0.2) (layer "F.Cu") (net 22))
 (segment (start 108.485 153.920001) (end 108.61 153.795001) (width 0.2) (layer "F.Cu") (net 22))
 (segment (start 108.61 153.795001) (end 108.61 153.45) (width 0.2) (layer "F.Cu") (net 22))
 (segment (start 108.51 156.75) (end 108.51 155.474999) (width 0.2) (layer "F.Cu") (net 22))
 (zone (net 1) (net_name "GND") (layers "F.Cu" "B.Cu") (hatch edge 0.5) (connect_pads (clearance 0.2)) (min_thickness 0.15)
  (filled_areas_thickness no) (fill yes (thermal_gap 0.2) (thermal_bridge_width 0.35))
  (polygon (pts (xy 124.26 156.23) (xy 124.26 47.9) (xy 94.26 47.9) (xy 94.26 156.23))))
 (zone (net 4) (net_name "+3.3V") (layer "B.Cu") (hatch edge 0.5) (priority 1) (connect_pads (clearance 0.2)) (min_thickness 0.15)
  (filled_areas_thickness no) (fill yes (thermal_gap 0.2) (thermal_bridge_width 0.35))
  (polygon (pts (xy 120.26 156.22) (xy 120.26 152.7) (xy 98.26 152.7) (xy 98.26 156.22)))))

